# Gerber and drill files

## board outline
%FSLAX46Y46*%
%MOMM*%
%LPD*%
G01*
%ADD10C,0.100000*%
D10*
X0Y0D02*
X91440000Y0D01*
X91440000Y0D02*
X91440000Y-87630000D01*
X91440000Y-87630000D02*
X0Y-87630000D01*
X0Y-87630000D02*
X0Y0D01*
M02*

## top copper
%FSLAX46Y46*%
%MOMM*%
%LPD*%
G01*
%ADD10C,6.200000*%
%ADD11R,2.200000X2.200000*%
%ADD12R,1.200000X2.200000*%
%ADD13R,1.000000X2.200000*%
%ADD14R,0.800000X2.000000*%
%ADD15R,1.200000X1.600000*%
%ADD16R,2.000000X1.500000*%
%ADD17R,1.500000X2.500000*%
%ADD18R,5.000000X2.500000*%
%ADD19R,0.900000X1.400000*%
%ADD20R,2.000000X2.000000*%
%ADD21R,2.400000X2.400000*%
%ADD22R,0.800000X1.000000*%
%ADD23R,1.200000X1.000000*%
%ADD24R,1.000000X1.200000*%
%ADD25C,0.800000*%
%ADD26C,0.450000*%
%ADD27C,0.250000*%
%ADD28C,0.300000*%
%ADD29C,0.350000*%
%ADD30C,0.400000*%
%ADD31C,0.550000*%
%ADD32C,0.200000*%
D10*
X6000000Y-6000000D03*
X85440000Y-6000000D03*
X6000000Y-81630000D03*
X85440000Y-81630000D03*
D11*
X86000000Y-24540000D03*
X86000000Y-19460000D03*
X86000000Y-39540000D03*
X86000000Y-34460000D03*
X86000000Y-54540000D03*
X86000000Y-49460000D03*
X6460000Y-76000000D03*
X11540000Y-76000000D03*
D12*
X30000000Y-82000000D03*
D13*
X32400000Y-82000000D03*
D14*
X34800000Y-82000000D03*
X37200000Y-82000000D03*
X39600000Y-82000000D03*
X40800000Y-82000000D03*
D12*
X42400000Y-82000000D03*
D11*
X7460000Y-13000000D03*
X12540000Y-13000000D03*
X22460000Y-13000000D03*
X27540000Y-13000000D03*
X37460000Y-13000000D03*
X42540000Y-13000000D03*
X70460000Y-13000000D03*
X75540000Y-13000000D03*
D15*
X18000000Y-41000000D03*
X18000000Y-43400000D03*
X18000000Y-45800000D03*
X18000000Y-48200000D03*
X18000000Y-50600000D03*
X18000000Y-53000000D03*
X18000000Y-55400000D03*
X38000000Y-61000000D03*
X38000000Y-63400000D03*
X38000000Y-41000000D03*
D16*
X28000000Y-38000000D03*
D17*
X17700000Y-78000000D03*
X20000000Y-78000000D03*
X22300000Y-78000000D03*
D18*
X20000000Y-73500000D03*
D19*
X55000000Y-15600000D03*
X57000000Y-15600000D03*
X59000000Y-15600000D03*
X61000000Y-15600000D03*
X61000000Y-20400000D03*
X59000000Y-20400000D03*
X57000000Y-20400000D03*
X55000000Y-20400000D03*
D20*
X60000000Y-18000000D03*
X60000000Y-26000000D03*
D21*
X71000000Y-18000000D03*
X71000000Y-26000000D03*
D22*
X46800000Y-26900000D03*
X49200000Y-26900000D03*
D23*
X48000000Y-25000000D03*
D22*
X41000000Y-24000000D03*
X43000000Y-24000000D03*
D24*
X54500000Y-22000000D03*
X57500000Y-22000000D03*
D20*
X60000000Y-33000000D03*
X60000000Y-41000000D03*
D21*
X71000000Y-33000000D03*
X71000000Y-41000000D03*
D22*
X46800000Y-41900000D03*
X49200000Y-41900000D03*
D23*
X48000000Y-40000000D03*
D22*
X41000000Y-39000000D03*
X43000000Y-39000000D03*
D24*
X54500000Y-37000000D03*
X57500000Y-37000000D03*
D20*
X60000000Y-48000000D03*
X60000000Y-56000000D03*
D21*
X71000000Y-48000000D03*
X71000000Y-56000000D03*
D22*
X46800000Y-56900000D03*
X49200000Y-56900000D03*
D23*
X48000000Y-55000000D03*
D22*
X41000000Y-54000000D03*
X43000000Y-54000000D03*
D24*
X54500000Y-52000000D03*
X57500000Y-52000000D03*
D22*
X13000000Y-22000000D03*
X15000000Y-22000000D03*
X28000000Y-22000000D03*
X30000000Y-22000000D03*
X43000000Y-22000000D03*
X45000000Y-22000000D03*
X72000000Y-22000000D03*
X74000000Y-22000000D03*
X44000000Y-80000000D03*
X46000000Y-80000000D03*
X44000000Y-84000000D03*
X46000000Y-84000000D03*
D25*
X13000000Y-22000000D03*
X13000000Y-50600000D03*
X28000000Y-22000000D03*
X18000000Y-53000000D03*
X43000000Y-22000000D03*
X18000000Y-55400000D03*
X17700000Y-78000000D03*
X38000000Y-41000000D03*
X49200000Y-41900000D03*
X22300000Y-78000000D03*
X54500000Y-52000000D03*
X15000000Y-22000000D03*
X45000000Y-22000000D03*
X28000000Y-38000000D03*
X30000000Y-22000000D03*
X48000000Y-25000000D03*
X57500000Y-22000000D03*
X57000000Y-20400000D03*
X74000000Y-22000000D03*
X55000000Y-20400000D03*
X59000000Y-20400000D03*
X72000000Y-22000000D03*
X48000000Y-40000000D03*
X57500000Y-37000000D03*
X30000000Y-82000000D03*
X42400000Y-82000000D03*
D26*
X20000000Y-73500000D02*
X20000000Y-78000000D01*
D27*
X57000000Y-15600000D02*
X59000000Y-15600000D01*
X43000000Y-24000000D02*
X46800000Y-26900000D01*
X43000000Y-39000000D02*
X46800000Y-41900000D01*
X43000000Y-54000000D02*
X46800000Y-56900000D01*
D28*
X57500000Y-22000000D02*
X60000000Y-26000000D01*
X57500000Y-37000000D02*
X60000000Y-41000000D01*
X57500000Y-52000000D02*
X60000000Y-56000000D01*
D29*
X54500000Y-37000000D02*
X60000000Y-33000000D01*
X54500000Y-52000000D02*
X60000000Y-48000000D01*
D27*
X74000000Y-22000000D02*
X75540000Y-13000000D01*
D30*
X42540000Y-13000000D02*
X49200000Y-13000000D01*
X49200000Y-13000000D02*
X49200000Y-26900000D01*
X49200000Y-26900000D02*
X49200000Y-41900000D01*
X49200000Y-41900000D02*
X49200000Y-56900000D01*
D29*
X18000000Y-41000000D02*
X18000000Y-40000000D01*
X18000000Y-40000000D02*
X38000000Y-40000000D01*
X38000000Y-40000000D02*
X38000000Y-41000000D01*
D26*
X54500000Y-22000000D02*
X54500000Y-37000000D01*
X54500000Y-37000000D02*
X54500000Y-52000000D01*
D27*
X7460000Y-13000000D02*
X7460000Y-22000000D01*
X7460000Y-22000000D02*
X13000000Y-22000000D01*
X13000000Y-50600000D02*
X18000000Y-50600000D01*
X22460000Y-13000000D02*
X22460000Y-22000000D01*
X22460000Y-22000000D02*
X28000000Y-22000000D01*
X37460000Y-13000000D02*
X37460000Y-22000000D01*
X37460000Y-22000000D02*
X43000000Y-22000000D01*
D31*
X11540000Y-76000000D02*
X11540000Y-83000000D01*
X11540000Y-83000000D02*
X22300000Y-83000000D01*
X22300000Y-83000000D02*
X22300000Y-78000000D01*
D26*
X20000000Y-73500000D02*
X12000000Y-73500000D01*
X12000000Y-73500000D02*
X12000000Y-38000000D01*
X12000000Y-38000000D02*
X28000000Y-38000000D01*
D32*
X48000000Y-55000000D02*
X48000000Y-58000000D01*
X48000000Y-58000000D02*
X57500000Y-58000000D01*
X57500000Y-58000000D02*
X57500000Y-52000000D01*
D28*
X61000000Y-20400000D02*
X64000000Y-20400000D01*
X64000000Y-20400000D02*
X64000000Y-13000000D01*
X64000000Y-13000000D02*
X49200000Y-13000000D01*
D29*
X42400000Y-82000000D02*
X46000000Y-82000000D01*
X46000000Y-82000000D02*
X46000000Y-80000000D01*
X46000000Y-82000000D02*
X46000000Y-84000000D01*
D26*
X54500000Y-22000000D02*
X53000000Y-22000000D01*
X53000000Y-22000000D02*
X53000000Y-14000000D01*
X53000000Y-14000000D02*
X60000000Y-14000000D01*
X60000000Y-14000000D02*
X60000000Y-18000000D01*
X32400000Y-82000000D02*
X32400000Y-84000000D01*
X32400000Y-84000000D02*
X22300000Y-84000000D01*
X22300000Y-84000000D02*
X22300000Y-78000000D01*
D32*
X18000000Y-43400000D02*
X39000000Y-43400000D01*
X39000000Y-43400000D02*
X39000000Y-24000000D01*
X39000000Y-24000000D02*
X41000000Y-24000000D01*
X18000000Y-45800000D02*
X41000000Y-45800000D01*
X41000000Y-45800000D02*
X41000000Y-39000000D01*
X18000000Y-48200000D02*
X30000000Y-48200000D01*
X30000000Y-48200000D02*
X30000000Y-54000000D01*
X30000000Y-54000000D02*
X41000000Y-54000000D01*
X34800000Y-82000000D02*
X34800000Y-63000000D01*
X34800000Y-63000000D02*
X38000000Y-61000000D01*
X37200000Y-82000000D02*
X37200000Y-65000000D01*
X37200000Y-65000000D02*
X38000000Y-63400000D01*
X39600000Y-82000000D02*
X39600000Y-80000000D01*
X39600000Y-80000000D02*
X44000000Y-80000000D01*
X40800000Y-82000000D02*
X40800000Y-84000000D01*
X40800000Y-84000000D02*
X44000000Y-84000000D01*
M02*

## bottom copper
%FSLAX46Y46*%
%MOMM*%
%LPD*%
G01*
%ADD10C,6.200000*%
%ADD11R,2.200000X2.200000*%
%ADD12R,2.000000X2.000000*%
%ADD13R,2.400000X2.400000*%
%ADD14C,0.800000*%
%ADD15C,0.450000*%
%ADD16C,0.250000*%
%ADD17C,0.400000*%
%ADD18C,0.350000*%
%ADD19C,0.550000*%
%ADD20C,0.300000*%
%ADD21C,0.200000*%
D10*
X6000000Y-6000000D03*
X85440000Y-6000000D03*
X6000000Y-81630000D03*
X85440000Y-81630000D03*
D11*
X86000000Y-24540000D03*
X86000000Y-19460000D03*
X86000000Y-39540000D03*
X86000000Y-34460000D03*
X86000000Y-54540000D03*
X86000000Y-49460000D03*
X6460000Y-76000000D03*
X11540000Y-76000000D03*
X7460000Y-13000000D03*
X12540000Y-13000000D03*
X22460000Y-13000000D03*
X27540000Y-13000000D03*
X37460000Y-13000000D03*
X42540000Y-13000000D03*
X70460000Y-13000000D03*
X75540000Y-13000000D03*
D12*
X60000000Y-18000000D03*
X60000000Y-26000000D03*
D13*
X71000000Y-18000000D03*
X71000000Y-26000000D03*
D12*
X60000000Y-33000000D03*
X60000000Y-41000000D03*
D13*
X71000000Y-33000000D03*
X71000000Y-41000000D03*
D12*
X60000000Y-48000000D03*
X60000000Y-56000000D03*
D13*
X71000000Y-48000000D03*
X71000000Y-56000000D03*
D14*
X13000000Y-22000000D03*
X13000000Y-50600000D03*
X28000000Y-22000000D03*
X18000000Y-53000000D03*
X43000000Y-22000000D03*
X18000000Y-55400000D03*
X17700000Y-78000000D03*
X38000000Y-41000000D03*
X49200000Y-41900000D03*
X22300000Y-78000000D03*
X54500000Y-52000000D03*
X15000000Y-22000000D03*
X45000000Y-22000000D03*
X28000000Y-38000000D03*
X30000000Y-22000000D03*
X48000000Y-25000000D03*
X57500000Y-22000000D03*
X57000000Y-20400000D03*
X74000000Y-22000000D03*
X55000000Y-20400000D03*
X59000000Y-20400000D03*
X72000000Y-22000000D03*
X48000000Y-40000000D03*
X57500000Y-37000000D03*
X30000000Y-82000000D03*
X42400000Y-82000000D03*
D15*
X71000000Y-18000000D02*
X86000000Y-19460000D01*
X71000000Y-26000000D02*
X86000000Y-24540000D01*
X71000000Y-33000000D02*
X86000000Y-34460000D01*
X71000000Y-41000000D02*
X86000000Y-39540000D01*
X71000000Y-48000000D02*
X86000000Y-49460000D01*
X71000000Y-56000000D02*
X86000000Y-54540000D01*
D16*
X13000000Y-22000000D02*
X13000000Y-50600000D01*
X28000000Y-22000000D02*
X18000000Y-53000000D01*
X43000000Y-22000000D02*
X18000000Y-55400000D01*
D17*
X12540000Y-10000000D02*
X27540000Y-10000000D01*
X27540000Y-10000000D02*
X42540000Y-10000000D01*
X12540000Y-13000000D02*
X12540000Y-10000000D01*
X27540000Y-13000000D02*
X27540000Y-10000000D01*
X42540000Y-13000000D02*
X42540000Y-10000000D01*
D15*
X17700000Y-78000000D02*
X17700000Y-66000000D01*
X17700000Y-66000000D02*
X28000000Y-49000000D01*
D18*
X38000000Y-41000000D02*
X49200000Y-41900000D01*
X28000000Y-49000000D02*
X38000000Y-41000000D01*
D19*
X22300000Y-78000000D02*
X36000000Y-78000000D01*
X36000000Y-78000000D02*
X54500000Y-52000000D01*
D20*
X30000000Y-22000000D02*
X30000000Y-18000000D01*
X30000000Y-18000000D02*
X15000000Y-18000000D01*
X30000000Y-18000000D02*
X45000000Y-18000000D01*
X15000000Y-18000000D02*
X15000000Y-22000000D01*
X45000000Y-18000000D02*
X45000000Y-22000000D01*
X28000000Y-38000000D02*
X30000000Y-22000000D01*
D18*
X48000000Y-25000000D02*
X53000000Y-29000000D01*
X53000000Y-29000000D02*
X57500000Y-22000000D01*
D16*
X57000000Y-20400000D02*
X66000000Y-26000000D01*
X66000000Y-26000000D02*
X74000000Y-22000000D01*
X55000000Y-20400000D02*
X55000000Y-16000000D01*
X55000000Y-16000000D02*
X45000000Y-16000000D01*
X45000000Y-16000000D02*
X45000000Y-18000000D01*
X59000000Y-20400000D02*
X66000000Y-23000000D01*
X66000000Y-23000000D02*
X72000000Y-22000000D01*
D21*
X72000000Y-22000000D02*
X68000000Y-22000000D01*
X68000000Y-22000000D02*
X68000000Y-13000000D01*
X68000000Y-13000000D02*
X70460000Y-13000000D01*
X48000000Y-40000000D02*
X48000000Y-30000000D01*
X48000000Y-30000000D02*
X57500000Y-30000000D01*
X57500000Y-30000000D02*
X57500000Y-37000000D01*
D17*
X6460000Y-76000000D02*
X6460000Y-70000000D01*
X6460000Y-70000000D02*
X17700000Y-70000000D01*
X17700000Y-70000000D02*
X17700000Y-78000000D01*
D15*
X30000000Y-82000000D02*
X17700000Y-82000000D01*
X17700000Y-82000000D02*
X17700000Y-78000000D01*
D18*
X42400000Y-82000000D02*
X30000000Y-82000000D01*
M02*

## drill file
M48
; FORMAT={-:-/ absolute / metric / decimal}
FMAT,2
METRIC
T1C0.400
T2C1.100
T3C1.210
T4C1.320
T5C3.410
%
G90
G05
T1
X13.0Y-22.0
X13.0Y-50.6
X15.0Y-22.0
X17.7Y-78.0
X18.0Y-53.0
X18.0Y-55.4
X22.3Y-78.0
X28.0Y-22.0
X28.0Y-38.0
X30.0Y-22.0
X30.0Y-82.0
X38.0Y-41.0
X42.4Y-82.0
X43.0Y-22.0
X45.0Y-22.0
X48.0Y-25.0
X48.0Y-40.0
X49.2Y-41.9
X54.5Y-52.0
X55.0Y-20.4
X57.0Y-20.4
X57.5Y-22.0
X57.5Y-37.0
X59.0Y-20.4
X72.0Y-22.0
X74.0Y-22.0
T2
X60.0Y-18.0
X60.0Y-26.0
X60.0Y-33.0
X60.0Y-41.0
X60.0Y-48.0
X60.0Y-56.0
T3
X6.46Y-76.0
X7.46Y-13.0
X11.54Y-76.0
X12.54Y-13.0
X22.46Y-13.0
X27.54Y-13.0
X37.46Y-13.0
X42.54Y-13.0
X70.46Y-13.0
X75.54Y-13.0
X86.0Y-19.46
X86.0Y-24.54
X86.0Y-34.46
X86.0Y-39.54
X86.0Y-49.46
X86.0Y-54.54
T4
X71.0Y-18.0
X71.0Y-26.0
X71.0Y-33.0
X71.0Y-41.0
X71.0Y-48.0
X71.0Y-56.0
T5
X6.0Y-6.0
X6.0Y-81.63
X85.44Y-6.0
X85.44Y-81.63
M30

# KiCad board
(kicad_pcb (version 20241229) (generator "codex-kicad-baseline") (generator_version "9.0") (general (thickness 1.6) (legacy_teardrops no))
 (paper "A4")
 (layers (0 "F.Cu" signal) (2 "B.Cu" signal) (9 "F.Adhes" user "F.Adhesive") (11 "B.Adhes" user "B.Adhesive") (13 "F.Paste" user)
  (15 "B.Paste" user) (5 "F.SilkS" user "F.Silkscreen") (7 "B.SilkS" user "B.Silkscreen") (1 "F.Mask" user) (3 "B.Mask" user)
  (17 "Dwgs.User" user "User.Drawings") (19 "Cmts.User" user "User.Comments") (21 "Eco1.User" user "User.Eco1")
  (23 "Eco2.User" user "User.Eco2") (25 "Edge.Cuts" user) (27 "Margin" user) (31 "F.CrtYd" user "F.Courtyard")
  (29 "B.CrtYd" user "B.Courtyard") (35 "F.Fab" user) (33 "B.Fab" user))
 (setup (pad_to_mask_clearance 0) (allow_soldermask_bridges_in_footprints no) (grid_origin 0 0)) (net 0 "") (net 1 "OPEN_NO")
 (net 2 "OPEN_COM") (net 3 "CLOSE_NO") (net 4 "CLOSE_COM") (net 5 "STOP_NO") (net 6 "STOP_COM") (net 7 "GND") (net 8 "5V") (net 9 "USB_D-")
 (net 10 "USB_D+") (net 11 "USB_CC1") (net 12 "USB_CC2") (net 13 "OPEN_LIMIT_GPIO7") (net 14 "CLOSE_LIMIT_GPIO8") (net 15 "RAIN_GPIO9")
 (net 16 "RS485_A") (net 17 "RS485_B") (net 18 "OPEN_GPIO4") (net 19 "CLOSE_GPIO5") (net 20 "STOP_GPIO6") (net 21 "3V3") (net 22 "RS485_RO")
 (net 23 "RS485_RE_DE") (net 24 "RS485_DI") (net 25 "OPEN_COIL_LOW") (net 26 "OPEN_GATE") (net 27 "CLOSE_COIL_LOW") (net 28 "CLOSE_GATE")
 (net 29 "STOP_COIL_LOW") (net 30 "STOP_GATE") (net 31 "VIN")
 (gr_line (start 0.00 0.00) (end 91.44 0.00) (stroke (width 0.1) (type solid)) (layer "Edge.Cuts"))
 (gr_line (start 91.44 0.00) (end 91.44 87.63) (stroke (width 0.1) (type solid)) (layer "Edge.Cuts"))
 (gr_line (start 91.44 87.63) (end 0.00 87.63) (stroke (width 0.1) (type solid)) (layer "Edge.Cuts"))
 (gr_line (start 0.00 87.63) (end 0.00 0.00) (stroke (width 0.1) (type solid)) (layer "Edge.Cuts"))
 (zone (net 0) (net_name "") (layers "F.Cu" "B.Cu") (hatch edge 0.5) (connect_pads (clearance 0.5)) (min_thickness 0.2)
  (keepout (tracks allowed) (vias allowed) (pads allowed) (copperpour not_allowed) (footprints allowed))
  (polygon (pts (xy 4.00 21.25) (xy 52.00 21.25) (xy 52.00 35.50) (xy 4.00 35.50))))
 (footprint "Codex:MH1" (layer "F.Cu") (at 6.00 6.00 0)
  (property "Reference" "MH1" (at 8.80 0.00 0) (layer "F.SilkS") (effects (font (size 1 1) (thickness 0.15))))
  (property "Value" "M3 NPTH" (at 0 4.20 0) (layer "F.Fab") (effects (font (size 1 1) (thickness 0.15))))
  (pad "1" np_thru_hole circle (at 0.00 0.00) (size 6.20 6.20) (drill 3.41) (layers "*.Cu" "*.Mask")))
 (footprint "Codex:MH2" (layer "F.Cu") (at 85.44 6.00 0)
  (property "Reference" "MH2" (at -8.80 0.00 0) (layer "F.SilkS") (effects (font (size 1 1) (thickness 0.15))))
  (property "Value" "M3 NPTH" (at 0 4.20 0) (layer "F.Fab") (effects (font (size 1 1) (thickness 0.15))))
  (pad "1" np_thru_hole circle (at 0.00 0.00) (size 6.20 6.20) (drill 3.41) (layers "*.Cu" "*.Mask")))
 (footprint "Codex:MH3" (layer "F.Cu") (at 6.00 81.63 0)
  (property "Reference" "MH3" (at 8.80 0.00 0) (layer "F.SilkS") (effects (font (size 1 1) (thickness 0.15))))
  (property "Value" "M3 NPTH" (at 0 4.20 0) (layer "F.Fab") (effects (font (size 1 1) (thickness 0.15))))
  (pad "1" np_thru_hole circle (at 0.00 0.00) (size 6.20 6.20) (drill 3.41) (layers "*.Cu" "*.Mask")))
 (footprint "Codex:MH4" (layer "F.Cu") (at 85.44 81.63 0)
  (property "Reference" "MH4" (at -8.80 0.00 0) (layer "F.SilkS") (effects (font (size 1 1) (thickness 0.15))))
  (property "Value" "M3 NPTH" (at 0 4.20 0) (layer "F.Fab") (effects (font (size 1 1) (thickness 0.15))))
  (pad "1" np_thru_hole circle (at 0.00 0.00) (size 6.20 6.20) (drill 3.41) (layers "*.Cu" "*.Mask")))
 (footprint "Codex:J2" (layer "F.Cu") (at 86.00 22.00 90)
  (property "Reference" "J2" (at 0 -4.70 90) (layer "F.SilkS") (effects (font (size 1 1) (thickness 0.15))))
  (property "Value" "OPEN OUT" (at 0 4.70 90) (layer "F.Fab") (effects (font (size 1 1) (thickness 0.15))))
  (pad "1" thru_hole rect (at -2.54 0.00) (size 2.20 2.20) (drill 1.21) (layers "*.Cu" "*.Mask") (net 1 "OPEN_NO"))
  (pad "2" thru_hole rect (at 2.54 0.00) (size 2.20 2.20) (drill 1.21) (layers "*.Cu" "*.Mask") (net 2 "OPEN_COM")))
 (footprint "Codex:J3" (layer "F.Cu") (at 86.00 37.00 90)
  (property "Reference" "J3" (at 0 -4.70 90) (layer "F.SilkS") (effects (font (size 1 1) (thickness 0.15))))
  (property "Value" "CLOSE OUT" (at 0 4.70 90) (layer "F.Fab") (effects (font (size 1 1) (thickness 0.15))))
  (pad "1" thru_hole rect (at -2.54 0.00) (size 2.20 2.20) (drill 1.21) (layers "*.Cu" "*.Mask") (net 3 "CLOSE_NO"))
  (pad "2" thru_hole rect (at 2.54 0.00) (size 2.20 2.20) (drill 1.21) (layers "*.Cu" "*.Mask") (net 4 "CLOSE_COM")))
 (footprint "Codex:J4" (layer "F.Cu") (at 86.00 52.00 90)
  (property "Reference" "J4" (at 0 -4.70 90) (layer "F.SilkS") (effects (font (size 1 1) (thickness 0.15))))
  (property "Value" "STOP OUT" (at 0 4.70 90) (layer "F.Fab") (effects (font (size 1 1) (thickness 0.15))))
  (pad "1" thru_hole rect (at -2.54 0.00) (size 2.20 2.20) (drill 1.21) (layers "*.Cu" "*.Mask") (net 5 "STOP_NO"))
  (pad "2" thru_hole rect (at 2.54 0.00) (size 2.20 2.20) (drill 1.21) (layers "*.Cu" "*.Mask") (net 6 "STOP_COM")))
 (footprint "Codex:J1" (layer "F.Cu") (at 9.00 76.00 0)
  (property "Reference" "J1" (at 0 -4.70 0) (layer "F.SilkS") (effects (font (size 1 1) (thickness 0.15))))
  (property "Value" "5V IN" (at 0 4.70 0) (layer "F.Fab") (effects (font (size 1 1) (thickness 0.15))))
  (pad "1" thru_hole rect (at -2.54 0.00) (size 2.20 2.20) (drill 1.21) (layers "*.Cu" "*.Mask") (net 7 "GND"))
  (pad "2" thru_hole rect (at 2.54 0.00) (size 2.20 2.20) (drill 1.21) (layers "*.Cu" "*.Mask") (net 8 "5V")))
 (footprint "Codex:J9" (layer "F.Cu") (at 36.00 82.00 0)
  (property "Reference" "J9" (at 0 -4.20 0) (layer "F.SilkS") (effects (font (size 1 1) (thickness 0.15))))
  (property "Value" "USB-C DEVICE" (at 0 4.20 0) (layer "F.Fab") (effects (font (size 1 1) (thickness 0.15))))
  (pad "GND1" smd rect (at -6.00 0.00) (size 1.20 2.20) (layers "F.Cu" "F.Paste" "F.Mask") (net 7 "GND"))
  (pad "VBUS" smd rect (at -3.60 0.00) (size 1.00 2.20) (layers "F.Cu" "F.Paste" "F.Mask") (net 8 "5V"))
  (pad "D-" smd rect (at -1.20 0.00) (size 0.80 2.00) (layers "F.Cu" "F.Paste" "F.Mask") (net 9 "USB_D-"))
  (pad "D+" smd rect (at 1.20 0.00) (size 0.80 2.00) (layers "F.Cu" "F.Paste" "F.Mask") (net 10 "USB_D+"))
  (pad "CC1" smd rect (at 3.60 0.00) (size 0.80 2.00) (layers "F.Cu" "F.Paste" "F.Mask") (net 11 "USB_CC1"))
  (pad "CC2" smd rect (at 4.80 0.00) (size 0.80 2.00) (layers "F.Cu" "F.Paste" "F.Mask") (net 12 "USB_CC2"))
  (pad "GND2" smd rect (at 6.40 0.00) (size 1.20 2.20) (layers "F.Cu" "F.Paste" "F.Mask") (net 7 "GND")))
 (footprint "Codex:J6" (layer "F.Cu") (at 10.00 13.00 0)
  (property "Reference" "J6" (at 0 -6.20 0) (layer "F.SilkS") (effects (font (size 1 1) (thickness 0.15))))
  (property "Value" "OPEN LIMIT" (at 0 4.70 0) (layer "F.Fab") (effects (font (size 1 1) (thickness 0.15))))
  (pad "1" thru_hole rect (at -2.54 0.00) (size 2.20 2.20) (drill 1.21) (layers "*.Cu" "*.Mask") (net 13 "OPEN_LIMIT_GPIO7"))
  (pad "2" thru_hole rect (at 2.54 0.00) (size 2.20 2.20) (drill 1.21) (layers "*.Cu" "*.Mask") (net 7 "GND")))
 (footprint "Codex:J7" (layer "F.Cu") (at 25.00 13.00 0)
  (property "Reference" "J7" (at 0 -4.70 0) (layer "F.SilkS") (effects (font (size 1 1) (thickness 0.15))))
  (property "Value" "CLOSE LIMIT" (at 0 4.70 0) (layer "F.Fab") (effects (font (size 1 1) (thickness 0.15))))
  (pad "1" thru_hole rect (at -2.54 0.00) (size 2.20 2.20) (drill 1.21) (layers "*.Cu" "*.Mask") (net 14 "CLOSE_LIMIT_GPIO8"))
  (pad "2" thru_hole rect (at 2.54 0.00) (size 2.20 2.20) (drill 1.21) (layers "*.Cu" "*.Mask") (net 7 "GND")))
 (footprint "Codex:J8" (layer "F.Cu") (at 40.00 13.00 0)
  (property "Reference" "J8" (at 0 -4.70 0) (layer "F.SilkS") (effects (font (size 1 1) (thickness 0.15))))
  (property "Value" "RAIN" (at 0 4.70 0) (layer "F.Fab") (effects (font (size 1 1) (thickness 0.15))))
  (pad "1" thru_hole rect (at -2.54 0.00) (size 2.20 2.20) (drill 1.21) (layers "*.Cu" "*.Mask") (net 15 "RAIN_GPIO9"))
  (pad "2" thru_hole rect (at 2.54 0.00) (size 2.20 2.20) (drill 1.21) (layers "*.Cu" "*.Mask") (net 7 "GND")))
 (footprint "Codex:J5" (layer "F.Cu") (at 73.00 13.00 0)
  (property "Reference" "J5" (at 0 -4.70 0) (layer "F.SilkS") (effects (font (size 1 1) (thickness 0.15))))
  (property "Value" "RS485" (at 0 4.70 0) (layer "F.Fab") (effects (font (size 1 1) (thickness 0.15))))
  (pad "1" thru_hole rect (at -2.54 0.00) (size 2.20 2.20) (drill 1.21) (layers "*.Cu" "*.Mask") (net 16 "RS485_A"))
  (pad "2" thru_hole rect (at 2.54 0.00) (size 2.20 2.20) (drill 1.21) (layers "*.Cu" "*.Mask") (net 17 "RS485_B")))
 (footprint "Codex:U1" (layer "F.Cu") (at 28.00 49.00 0)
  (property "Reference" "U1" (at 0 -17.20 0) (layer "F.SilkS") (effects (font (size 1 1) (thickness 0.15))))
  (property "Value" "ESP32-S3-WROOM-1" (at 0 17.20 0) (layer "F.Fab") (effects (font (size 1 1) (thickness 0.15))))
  (pad "1" smd rect (at -10.00 -8.00) (size 1.20 1.60) (layers "F.Cu" "F.Paste" "F.Mask") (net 7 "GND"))
  (pad "4" smd rect (at -10.00 -5.60) (size 1.20 1.60) (layers "F.Cu" "F.Paste" "F.Mask") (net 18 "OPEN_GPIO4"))
  (pad "5" smd rect (at -10.00 -3.20) (size 1.20 1.60) (layers "F.Cu" "F.Paste" "F.Mask") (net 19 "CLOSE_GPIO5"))
  (pad "6" smd rect (at -10.00 -0.80) (size 1.20 1.60) (layers "F.Cu" "F.Paste" "F.Mask") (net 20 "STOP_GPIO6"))
  (pad "7" smd rect (at -10.00 1.60) (size 1.20 1.60) (layers "F.Cu" "F.Paste" "F.Mask") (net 13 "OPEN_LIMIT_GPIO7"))
  (pad "12" smd rect (at -10.00 4.00) (size 1.20 1.60) (layers "F.Cu" "F.Paste" "F.Mask") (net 14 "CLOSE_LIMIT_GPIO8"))
  (pad "17" smd rect (at -10.00 6.40) (size 1.20 1.60) (layers "F.Cu" "F.Paste" "F.Mask") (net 15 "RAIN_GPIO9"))
  (pad "19" smd rect (at 10.00 12.00) (size 1.20 1.60) (layers "F.Cu" "F.Paste" "F.Mask") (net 9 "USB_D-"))
  (pad "20" smd rect (at 10.00 14.40) (size 1.20 1.60) (layers "F.Cu" "F.Paste" "F.Mask") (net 10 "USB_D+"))
  (pad "40" smd rect (at 10.00 -8.00) (size 1.20 1.60) (layers "F.Cu" "F.Paste" "F.Mask") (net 7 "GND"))
  (pad "3V3" smd rect (at 0.00 -11.00) (size 2.00 1.50) (layers "F.Cu" "F.Paste" "F.Mask") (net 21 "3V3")))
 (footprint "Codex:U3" (layer "F.Cu") (at 20.00 76.00 0)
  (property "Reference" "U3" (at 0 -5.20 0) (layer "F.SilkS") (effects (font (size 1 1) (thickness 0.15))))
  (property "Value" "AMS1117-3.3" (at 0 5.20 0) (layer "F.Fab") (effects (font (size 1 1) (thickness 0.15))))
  (pad "1" smd rect (at -2.30 2.00) (size 1.50 2.50) (layers "F.Cu" "F.Paste" "F.Mask") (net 7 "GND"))
  (pad "2" smd rect (at 0.00 2.00) (size 1.50 2.50) (layers "F.Cu" "F.Paste" "F.Mask") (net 21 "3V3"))
  (pad "3" smd rect (at 2.30 2.00) (size 1.50 2.50) (layers "F.Cu" "F.Paste" "F.Mask") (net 8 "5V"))
  (pad "4" smd rect (at 0.00 -2.50) (size 5.00 2.50) (layers "F.Cu" "F.Paste" "F.Mask") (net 21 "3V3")))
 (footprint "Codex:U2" (layer "F.Cu") (at 58.00 18.00 0)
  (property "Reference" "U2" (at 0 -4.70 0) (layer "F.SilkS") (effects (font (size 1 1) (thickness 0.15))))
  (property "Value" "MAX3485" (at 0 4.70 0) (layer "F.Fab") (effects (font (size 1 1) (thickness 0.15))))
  (pad "1" smd rect (at -3.00 -2.40) (size 0.90 1.40) (layers "F.Cu" "F.Paste" "F.Mask") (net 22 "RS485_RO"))
  (pad "2" smd rect (at -1.00 -2.40) (size 0.90 1.40) (layers "F.Cu" "F.Paste" "F.Mask") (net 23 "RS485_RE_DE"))
  (pad "3" smd rect (at 1.00 -2.40) (size 0.90 1.40) (layers "F.Cu" "F.Paste" "F.Mask") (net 23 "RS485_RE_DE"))
  (pad "4" smd rect (at 3.00 -2.40) (size 0.90 1.40) (layers "F.Cu" "F.Paste" "F.Mask") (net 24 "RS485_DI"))
  (pad "5" smd rect (at 3.00 2.40) (size 0.90 1.40) (layers "F.Cu" "F.Paste" "F.Mask") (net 7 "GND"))
  (pad "6" smd rect (at 1.00 2.40) (size 0.90 1.40) (layers "F.Cu" "F.Paste" "F.Mask") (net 16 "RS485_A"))
  (pad "7" smd rect (at -1.00 2.40) (size 0.90 1.40) (layers "F.Cu" "F.Paste" "F.Mask") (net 17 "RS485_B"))
  (pad "8" smd rect (at -3.00 2.40) (size 0.90 1.40) (layers "F.Cu" "F.Paste" "F.Mask") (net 21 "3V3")))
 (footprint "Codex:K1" (layer "F.Cu") (at 66.00 22.00 0)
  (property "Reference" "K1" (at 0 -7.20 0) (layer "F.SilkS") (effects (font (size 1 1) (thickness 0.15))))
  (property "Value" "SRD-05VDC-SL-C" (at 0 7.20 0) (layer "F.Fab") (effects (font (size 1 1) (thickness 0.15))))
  (pad "COIL+" thru_hole rect (at -6.00 -4.00) (size 2.00 2.00) (drill 1.10) (layers "*.Cu" "*.Mask") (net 8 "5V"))
  (pad "COIL-" thru_hole rect (at -6.00 4.00) (size 2.00 2.00) (drill 1.10) (layers "*.Cu" "*.Mask") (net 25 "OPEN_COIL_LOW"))
  (pad "COM" thru_hole rect (at 5.00 -4.00) (size 2.40 2.40) (drill 1.32) (layers "*.Cu" "*.Mask") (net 2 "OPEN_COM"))
  (pad "NO" thru_hole rect (at 5.00 4.00) (size 2.40 2.40) (drill 1.32) (layers "*.Cu" "*.Mask") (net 1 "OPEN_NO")))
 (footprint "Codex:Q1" (layer "F.Cu") (at 48.00 26.00 0)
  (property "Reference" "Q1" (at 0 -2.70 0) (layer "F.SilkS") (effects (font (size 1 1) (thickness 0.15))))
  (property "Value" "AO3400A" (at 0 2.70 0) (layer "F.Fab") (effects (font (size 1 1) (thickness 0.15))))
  (pad "1" smd rect (at -1.20 0.90) (size 0.80 1.00) (layers "F.Cu" "F.Paste" "F.Mask") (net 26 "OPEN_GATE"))
  (pad "2" smd rect (at 1.20 0.90) (size 0.80 1.00) (layers "F.Cu" "F.Paste" "F.Mask") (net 7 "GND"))
  (pad "3" smd rect (at 0.00 -1.00) (size 1.20 1.00) (layers "F.Cu" "F.Paste" "F.Mask") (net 25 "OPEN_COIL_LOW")))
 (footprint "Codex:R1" (layer "F.Cu") (at 42.00 24.00 0)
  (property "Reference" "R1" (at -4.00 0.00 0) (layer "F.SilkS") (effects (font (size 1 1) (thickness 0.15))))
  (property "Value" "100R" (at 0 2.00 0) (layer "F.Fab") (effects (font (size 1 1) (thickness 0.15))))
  (pad "1" smd rect (at -1.00 0.00) (size 0.80 1.00) (layers "F.Cu" "F.Paste" "F.Mask") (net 18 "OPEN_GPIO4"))
  (pad "2" smd rect (at 1.00 0.00) (size 0.80 1.00) (layers "F.Cu" "F.Paste" "F.Mask") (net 26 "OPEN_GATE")))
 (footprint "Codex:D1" (layer "F.Cu") (at 56.00 22.00 0)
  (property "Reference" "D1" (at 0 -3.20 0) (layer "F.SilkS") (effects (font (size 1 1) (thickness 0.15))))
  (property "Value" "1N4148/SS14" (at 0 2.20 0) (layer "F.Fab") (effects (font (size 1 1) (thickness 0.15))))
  (pad "1" smd rect (at -1.50 0.00) (size 1.00 1.20) (layers "F.Cu" "F.Paste" "F.Mask") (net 8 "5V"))
  (pad "2" smd rect (at 1.50 0.00) (size 1.00 1.20) (layers "F.Cu" "F.Paste" "F.Mask") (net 25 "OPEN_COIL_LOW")))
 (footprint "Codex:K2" (layer "F.Cu") (at 66.00 37.00 0)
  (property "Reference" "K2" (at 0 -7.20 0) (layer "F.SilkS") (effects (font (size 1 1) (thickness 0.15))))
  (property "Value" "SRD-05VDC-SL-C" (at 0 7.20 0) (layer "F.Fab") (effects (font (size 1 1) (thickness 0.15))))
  (pad "COIL+" thru_hole rect (at -6.00 -4.00) (size 2.00 2.00) (drill 1.10) (layers "*.Cu" "*.Mask") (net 8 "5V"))
  (pad "COIL-" thru_hole rect (at -6.00 4.00) (size 2.00 2.00) (drill 1.10) (layers "*.Cu" "*.Mask") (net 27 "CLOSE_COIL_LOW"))
  (pad "COM" thru_hole rect (at 5.00 -4.00) (size 2.40 2.40) (drill 1.32) (layers "*.Cu" "*.Mask") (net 4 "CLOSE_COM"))
  (pad "NO" thru_hole rect (at 5.00 4.00) (size 2.40 2.40) (drill 1.32) (layers "*.Cu" "*.Mask") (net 3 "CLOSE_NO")))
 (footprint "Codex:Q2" (layer "F.Cu") (at 48.00 41.00 0)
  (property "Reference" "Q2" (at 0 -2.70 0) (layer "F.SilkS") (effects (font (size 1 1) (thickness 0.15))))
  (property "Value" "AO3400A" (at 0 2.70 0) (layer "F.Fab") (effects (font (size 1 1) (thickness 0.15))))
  (pad "1" smd rect (at -1.20 0.90) (size 0.80 1.00) (layers "F.Cu" "F.Paste" "F.Mask") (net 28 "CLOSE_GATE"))
  (pad "2" smd rect (at 1.20 0.90) (size 0.80 1.00) (layers "F.Cu" "F.Paste" "F.Mask") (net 7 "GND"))
  (pad "3" smd rect (at 0.00 -1.00) (size 1.20 1.00) (layers "F.Cu" "F.Paste" "F.Mask") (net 27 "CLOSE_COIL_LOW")))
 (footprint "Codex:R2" (layer "F.Cu") (at 42.00 39.00 0)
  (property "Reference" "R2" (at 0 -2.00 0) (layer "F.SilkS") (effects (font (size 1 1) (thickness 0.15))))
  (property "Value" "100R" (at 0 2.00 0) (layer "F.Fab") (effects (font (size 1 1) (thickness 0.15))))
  (pad "1" smd rect (at -1.00 0.00) (size 0.80 1.00) (layers "F.Cu" "F.Paste" "F.Mask") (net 19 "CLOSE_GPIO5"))
  (pad "2" smd rect (at 1.00 0.00) (size 0.80 1.00) (layers "F.Cu" "F.Paste" "F.Mask") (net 28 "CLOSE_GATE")))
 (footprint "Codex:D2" (layer "F.Cu") (at 56.00 37.00 0)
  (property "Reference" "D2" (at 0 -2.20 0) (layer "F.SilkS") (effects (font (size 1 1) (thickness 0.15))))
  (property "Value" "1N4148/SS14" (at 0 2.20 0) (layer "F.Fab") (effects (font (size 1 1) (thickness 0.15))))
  (pad "1" smd rect (at -1.50 0.00) (size 1.00 1.20) (layers "F.Cu" "F.Paste" "F.Mask") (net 8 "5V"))
  (pad "2" smd rect (at 1.50 0.00) (size 1.00 1.20) (layers "F.Cu" "F.Paste" "F.Mask") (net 27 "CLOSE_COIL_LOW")))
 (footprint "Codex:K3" (layer "F.Cu") (at 66.00 52.00 0)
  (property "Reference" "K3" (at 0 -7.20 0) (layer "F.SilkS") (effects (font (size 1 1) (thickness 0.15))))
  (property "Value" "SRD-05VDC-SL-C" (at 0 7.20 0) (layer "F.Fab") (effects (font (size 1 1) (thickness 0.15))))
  (pad "COIL+" thru_hole rect (at -6.00 -4.00) (size 2.00 2.00) (drill 1.10) (layers "*.Cu" "*.Mask") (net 8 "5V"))
  (pad "COIL-" thru_hole rect (at -6.00 4.00) (size 2.00 2.00) (drill 1.10) (layers "*.Cu" "*.Mask") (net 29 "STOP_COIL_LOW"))
  (pad "COM" thru_hole rect (at 5.00 -4.00) (size 2.40 2.40) (drill 1.32) (layers "*.Cu" "*.Mask") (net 6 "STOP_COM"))
  (pad "NO" thru_hole rect (at 5.00 4.00) (size 2.40 2.40) (drill 1.32) (layers "*.Cu" "*.Mask") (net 5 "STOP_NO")))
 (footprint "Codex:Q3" (layer "F.Cu") (at 48.00 56.00 0)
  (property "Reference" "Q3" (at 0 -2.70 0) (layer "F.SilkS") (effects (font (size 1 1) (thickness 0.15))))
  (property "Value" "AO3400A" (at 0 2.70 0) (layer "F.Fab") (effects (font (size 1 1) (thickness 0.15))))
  (pad "1" smd rect (at -1.20 0.90) (size 0.80 1.00) (layers "F.Cu" "F.Paste" "F.Mask") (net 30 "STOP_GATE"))
  (pad "2" smd rect (at 1.20 0.90) (size 0.80 1.00) (layers "F.Cu" "F.Paste" "F.Mask") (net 7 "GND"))
  (pad "3" smd rect (at 0.00 -1.00) (size 1.20 1.00) (layers "F.Cu" "F.Paste" "F.Mask") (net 29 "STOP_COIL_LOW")))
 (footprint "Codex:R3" (layer "F.Cu") (at 42.00 54.00 0)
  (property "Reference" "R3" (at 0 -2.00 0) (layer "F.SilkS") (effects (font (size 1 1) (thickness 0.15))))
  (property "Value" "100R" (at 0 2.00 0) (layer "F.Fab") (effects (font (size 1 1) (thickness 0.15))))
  (pad "1" smd rect (at -1.00 0.00) (size 0.80 1.00) (layers "F.Cu" "F.Paste" "F.Mask") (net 20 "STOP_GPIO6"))
  (pad "2" smd rect (at 1.00 0.00) (size 0.80 1.00) (layers "F.Cu" "F.Paste" "F.Mask") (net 30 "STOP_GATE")))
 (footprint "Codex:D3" (layer "F.Cu") (at 56.00 52.00 0)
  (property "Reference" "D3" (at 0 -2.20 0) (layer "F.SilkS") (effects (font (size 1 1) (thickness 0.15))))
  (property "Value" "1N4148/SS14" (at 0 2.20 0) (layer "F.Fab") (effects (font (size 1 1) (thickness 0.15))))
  (pad "1" smd rect (at -1.50 0.00) (size 1.00 1.20) (layers "F.Cu" "F.Paste" "F.Mask") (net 8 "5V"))
  (pad "2" smd rect (at 1.50 0.00) (size 1.00 1.20) (layers "F.Cu" "F.Paste" "F.Mask") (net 29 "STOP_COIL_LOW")))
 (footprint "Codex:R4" (layer "F.Cu") (at 14.00 22.00 0)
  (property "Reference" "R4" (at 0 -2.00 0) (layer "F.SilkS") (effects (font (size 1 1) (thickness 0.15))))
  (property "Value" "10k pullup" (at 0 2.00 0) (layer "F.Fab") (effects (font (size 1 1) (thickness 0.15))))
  (pad "1" smd rect (at -1.00 0.00) (size 0.80 1.00) (layers "F.Cu" "F.Paste" "F.Mask") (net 13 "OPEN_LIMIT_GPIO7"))
  (pad "2" smd rect (at 1.00 0.00) (size 0.80 1.00) (layers "F.Cu" "F.Paste" "F.Mask") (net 21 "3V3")))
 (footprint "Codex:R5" (layer "F.Cu") (at 29.00 22.00 0)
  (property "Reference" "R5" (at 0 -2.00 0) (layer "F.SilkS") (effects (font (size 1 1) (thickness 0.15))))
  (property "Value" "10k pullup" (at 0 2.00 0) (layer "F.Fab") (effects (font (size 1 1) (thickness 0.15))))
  (pad "1" smd rect (at -1.00 0.00) (size 0.80 1.00) (layers "F.Cu" "F.Paste" "F.Mask") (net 14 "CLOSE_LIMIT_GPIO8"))
  (pad "2" smd rect (at 1.00 0.00) (size 0.80 1.00) (layers "F.Cu" "F.Paste" "F.Mask") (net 21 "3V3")))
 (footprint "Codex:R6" (layer "F.Cu") (at 44.00 22.00 0)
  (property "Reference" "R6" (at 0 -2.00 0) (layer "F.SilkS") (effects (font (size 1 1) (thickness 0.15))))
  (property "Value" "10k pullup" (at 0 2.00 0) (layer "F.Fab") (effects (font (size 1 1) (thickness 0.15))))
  (pad "1" smd rect (at -1.00 0.00) (size 0.80 1.00) (layers "F.Cu" "F.Paste" "F.Mask") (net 15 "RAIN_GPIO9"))
  (pad "2" smd rect (at 1.00 0.00) (size 0.80 1.00) (layers "F.Cu" "F.Paste" "F.Mask") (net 21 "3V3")))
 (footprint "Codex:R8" (layer "F.Cu") (at 73.00 22.00 0)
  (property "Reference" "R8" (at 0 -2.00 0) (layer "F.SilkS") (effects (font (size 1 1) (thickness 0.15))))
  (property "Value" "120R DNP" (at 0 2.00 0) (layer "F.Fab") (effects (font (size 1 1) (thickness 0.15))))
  (pad "1" smd rect (at -1.00 0.00) (size 0.80 1.00) (layers "F.Cu" "F.Paste" "F.Mask") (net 16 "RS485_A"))
  (pad "2" smd rect (at 1.00 0.00) (size 0.80 1.00) (layers "F.Cu" "F.Paste" "F.Mask") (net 17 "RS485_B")))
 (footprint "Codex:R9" (layer "F.Cu") (at 45.00 80.00 0)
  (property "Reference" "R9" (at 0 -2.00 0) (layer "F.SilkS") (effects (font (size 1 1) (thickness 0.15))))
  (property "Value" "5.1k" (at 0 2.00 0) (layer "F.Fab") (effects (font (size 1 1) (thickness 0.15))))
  (pad "1" smd rect (at -1.00 0.00) (size 0.80 1.00) (layers "F.Cu" "F.Paste" "F.Mask") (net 11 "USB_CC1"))
  (pad "2" smd rect (at 1.00 0.00) (size 0.80 1.00) (layers "F.Cu" "F.Paste" "F.Mask") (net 7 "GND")))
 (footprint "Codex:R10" (layer "F.Cu") (at 45.00 84.00 0)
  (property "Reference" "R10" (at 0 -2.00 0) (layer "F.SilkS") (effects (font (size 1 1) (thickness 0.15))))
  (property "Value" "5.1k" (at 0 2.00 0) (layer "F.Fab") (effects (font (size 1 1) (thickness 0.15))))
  (pad "1" smd rect (at -1.00 0.00) (size 0.80 1.00) (layers "F.Cu" "F.Paste" "F.Mask") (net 12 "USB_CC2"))
  (pad "2" smd rect (at 1.00 0.00) (size 0.80 1.00) (layers "F.Cu" "F.Paste" "F.Mask") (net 7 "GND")))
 (segment (start 71.00 18.00) (end 86.00 19.46) (width 0.45) (layer "B.Cu") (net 2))
 (segment (start 71.00 26.00) (end 86.00 24.54) (width 0.45) (layer "B.Cu") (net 1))
 (segment (start 71.00 33.00) (end 86.00 34.46) (width 0.45) (layer "B.Cu") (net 4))
 (segment (start 71.00 41.00) (end 86.00 39.54) (width 0.45) (layer "B.Cu") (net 3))
 (segment (start 71.00 48.00) (end 86.00 49.46) (width 0.45) (layer "B.Cu") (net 6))
 (segment (start 71.00 56.00) (end 86.00 54.54) (width 0.45) (layer "B.Cu") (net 5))
 (segment (start 20.00 73.50) (end 20.00 78.00) (width 0.45) (layer "F.Cu") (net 21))
 (segment (start 57.00 15.60) (end 59.00 15.60) (width 0.25) (layer "F.Cu") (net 23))
 (segment (start 43.00 24.00) (end 46.80 26.90) (width 0.25) (layer "F.Cu") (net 26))
 (segment (start 43.00 39.00) (end 46.80 41.90) (width 0.25) (layer "F.Cu") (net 28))
 (segment (start 43.00 54.00) (end 46.80 56.90) (width 0.25) (layer "F.Cu") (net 30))
 (segment (start 57.50 22.00) (end 60.00 26.00) (width 0.30) (layer "F.Cu") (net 25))
 (segment (start 57.50 37.00) (end 60.00 41.00) (width 0.30) (layer "F.Cu") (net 27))
 (segment (start 57.50 52.00) (end 60.00 56.00) (width 0.30) (layer "F.Cu") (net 29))
 (segment (start 54.50 37.00) (end 60.00 33.00) (width 0.35) (layer "F.Cu") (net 8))
 (segment (start 54.50 52.00) (end 60.00 48.00) (width 0.35) (layer "F.Cu") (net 8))
 (segment (start 74.00 22.00) (end 75.54 13.00) (width 0.25) (layer "F.Cu") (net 17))
 (segment (start 42.54 13.00) (end 49.20 13.00) (width 0.40) (layer "F.Cu") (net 7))
 (segment (start 49.20 13.00) (end 49.20 26.90) (width 0.40) (layer "F.Cu") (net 7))
 (segment (start 49.20 26.90) (end 49.20 41.90) (width 0.40) (layer "F.Cu") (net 7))
 (segment (start 49.20 41.90) (end 49.20 56.90) (width 0.40) (layer "F.Cu") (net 7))
 (segment (start 18.00 41.00) (end 18.00 40.00) (width 0.35) (layer "F.Cu") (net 7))
 (segment (start 18.00 40.00) (end 38.00 40.00) (width 0.35) (layer "F.Cu") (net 7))
 (segment (start 38.00 40.00) (end 38.00 41.00) (width 0.35) (layer "F.Cu") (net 7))
 (segment (start 54.50 22.00) (end 54.50 37.00) (width 0.45) (layer "F.Cu") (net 8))
 (segment (start 54.50 37.00) (end 54.50 52.00) (width 0.45) (layer "F.Cu") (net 8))
 (segment (start 7.46 13.00) (end 7.46 22.00) (width 0.25) (layer "F.Cu") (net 13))
 (segment (start 7.46 22.00) (end 13.00 22.00) (width 0.25) (layer "F.Cu") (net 13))
 (segment (start 13.00 22.00) (end 13.00 50.60) (width 0.25) (layer "B.Cu") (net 13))
 (via (at 13.00 22.00) (size 0.80) (drill 0.40) (layers "F.Cu" "B.Cu") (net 13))
 (via (at 13.00 50.60) (size 0.80) (drill 0.40) (layers "F.Cu" "B.Cu") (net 13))
 (segment (start 13.00 50.60) (end 18.00 50.60) (width 0.25) (layer "F.Cu") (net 13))
 (segment (start 22.46 13.00) (end 22.46 22.00) (width 0.25) (layer "F.Cu") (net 14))
 (segment (start 22.46 22.00) (end 28.00 22.00) (width 0.25) (layer "F.Cu") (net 14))
 (segment (start 28.00 22.00) (end 18.00 53.00) (width 0.25) (layer "B.Cu") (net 14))
 (via (at 28.00 22.00) (size 0.80) (drill 0.40) (layers "F.Cu" "B.Cu") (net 14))
 (via (at 18.00 53.00) (size 0.80) (drill 0.40) (layers "F.Cu" "B.Cu") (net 14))
 (segment (start 37.46 13.00) (end 37.46 22.00) (width 0.25) (layer "F.Cu") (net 15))
 (segment (start 37.46 22.00) (end 43.00 22.00) (width 0.25) (layer "F.Cu") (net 15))
 (segment (start 43.00 22.00) (end 18.00 55.40) (width 0.25) (layer "B.Cu") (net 15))
 (via (at 43.00 22.00) (size 0.80) (drill 0.40) (layers "F.Cu" "B.Cu") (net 15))
 (via (at 18.00 55.40) (size 0.80) (drill 0.40) (layers "F.Cu" "B.Cu") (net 15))
 (segment (start 12.54 10.00) (end 27.54 10.00) (width 0.40) (layer "B.Cu") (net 7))
 (segment (start 27.54 10.00) (end 42.54 10.00) (width 0.40) (layer "B.Cu") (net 7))
 (segment (start 12.54 13.00) (end 12.54 10.00) (width 0.40) (layer "B.Cu") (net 7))
 (segment (start 27.54 13.00) (end 27.54 10.00) (width 0.40) (layer "B.Cu") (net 7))
 (segment (start 42.54 13.00) (end 42.54 10.00) (width 0.40) (layer "B.Cu") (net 7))
 (via (at 17.70 78.00) (size 0.80) (drill 0.40) (layers "F.Cu" "B.Cu") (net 7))
 (segment (start 17.70 78.00) (end 17.70 66.00) (width 0.45) (layer "B.Cu") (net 7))
 (segment (start 17.70 66.00) (end 28.00 49.00) (width 0.45) (layer "B.Cu") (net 7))
 (via (at 38.00 41.00) (size 0.80) (drill 0.40) (layers "F.Cu" "B.Cu") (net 7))
 (segment (start 38.00 41.00) (end 49.20 41.90) (width 0.35) (layer "B.Cu") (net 7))
 (via (at 49.20 41.90) (size 0.80) (drill 0.40) (layers "F.Cu" "B.Cu") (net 7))
 (segment (start 28.00 49.00) (end 38.00 41.00) (width 0.35) (layer "B.Cu") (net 7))
 (segment (start 11.54 76.00) (end 11.54 83.00) (width 0.55) (layer "F.Cu") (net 8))
 (segment (start 11.54 83.00) (end 22.30 83.00) (width 0.55) (layer "F.Cu") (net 8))
 (segment (start 22.30 83.00) (end 22.30 78.00) (width 0.55) (layer "F.Cu") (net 8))
 (via (at 22.30 78.00) (size 0.80) (drill 0.40) (layers "F.Cu" "B.Cu") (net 8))
 (segment (start 22.30 78.00) (end 36.00 78.00) (width 0.55) (layer "B.Cu") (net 8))
 (segment (start 36.00 78.00) (end 54.50 52.00) (width 0.55) (layer "B.Cu") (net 8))
 (via (at 54.50 52.00) (size 0.80) (drill 0.40) (layers "F.Cu" "B.Cu") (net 8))
 (segment (start 30.00 22.00) (end 30.00 18.00) (width 0.30) (layer "B.Cu") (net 21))
 (segment (start 30.00 18.00) (end 15.00 18.00) (width 0.30) (layer "B.Cu") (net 21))
 (segment (start 30.00 18.00) (end 45.00 18.00) (width 0.30) (layer "B.Cu") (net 21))
 (via (at 15.00 22.00) (size 0.80) (drill 0.40) (layers "F.Cu" "B.Cu") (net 21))
 (segment (start 15.00 18.00) (end 15.00 22.00) (width 0.30) (layer "B.Cu") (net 21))
 (via (at 45.00 22.00) (size 0.80) (drill 0.40) (layers "F.Cu" "B.Cu") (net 21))
 (segment (start 45.00 18.00) (end 45.00 22.00) (width 0.30) (layer "B.Cu") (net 21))
 (via (at 28.00 38.00) (size 0.80) (drill 0.40) (layers "F.Cu" "B.Cu") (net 21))
 (segment (start 28.00 38.00) (end 30.00 22.00) (width 0.30) (layer "B.Cu") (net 21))
 (via (at 30.00 22.00) (size 0.80) (drill 0.40) (layers "F.Cu" "B.Cu") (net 21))
 (via (at 48.00 25.00) (size 0.80) (drill 0.40) (layers "F.Cu" "B.Cu") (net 25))
 (segment (start 48.00 25.00) (end 53.00 29.00) (width 0.35) (layer "B.Cu") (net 25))
 (segment (start 53.00 29.00) (end 57.50 22.00) (width 0.35) (layer "B.Cu") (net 25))
 (via (at 57.50 22.00) (size 0.80) (drill 0.40) (layers "F.Cu" "B.Cu") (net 25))
 (via (at 57.00 20.40) (size 0.80) (drill 0.40) (layers "F.Cu" "B.Cu") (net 17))
 (segment (start 57.00 20.40) (end 66.00 26.00) (width 0.25) (layer "B.Cu") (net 17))
 (segment (start 66.00 26.00) (end 74.00 22.00) (width 0.25) (layer "B.Cu") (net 17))
 (via (at 74.00 22.00) (size 0.80) (drill 0.40) (layers "F.Cu" "B.Cu") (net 17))
 (segment (start 20.00 73.50) (end 12.00 73.50) (width 0.45) (layer "F.Cu") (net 21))
 (segment (start 12.00 73.50) (end 12.00 38.00) (width 0.45) (layer "F.Cu") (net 21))
 (segment (start 12.00 38.00) (end 28.00 38.00) (width 0.45) (layer "F.Cu") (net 21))
 (via (at 55.00 20.40) (size 0.80) (drill 0.40) (layers "F.Cu" "B.Cu") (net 21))
 (segment (start 55.00 20.40) (end 55.00 16.00) (width 0.25) (layer "B.Cu") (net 21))
 (segment (start 55.00 16.00) (end 45.00 16.00) (width 0.25) (layer "B.Cu") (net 21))
 (segment (start 45.00 16.00) (end 45.00 18.00) (width 0.25) (layer "B.Cu") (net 21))
 (via (at 59.00 20.40) (size 0.80) (drill 0.40) (layers "F.Cu" "B.Cu") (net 16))
 (segment (start 59.00 20.40) (end 66.00 23.00) (width 0.25) (layer "B.Cu") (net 16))
 (segment (start 66.00 23.00) (end 72.00 22.00) (width 0.25) (layer "B.Cu") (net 16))
 (via (at 72.00 22.00) (size 0.80) (drill 0.40) (layers "F.Cu" "B.Cu") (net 16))
 (segment (start 72.00 22.00) (end 68.00 22.00) (width 0.20) (layer "B.Cu") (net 16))
 (segment (start 68.00 22.00) (end 68.00 13.00) (width 0.20) (layer "B.Cu") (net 16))
 (segment (start 68.00 13.00) (end 70.46 13.00) (width 0.20) (layer "B.Cu") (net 16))
 (via (at 48.00 40.00) (size 0.80) (drill 0.40) (layers "F.Cu" "B.Cu") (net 27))
 (via (at 57.50 37.00) (size 0.80) (drill 0.40) (layers "F.Cu" "B.Cu") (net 27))
 (segment (start 48.00 40.00) (end 48.00 30.00) (width 0.20) (layer "B.Cu") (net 27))
 (segment (start 48.00 30.00) (end 57.50 30.00) (width 0.20) (layer "B.Cu") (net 27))
 (segment (start 57.50 30.00) (end 57.50 37.00) (width 0.20) (layer "B.Cu") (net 27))
 (segment (start 48.00 55.00) (end 48.00 58.00) (width 0.20) (layer "F.Cu") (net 29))
 (segment (start 48.00 58.00) (end 57.50 58.00) (width 0.20) (layer "F.Cu") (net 29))
 (segment (start 57.50 58.00) (end 57.50 52.00) (width 0.20) (layer "F.Cu") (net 29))
 (segment (start 6.46 76.00) (end 6.46 70.00) (width 0.40) (layer "B.Cu") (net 7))
 (segment (start 6.46 70.00) (end 17.70 70.00) (width 0.40) (layer "B.Cu") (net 7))
 (segment (start 17.70 70.00) (end 17.70 78.00) (width 0.40) (layer "B.Cu") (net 7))
 (segment (start 61.00 20.40) (end 64.00 20.40) (width 0.30) (layer "F.Cu") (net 7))
 (segment (start 64.00 20.40) (end 64.00 13.00) (width 0.30) (layer "F.Cu") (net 7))
 (segment (start 64.00 13.00) (end 49.20 13.00) (width 0.30) (layer "F.Cu") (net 7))
 (segment (start 30.00 82.00) (end 17.70 82.00) (width 0.45) (layer "B.Cu") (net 7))
 (segment (start 17.70 82.00) (end 17.70 78.00) (width 0.45) (layer "B.Cu") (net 7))
 (via (at 30.00 82.00) (size 0.80) (drill 0.40) (layers "F.Cu" "B.Cu") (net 7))
 (via (at 42.40 82.00) (size 0.80) (drill 0.40) (layers "F.Cu" "B.Cu") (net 7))
 (segment (start 42.40 82.00) (end 30.00 82.00) (width 0.35) (layer "B.Cu") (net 7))
 (segment (start 42.40 82.00) (end 46.00 82.00) (width 0.35) (layer "F.Cu") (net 7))
 (segment (start 46.00 82.00) (end 46.00 80.00) (width 0.35) (layer "F.Cu") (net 7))
 (segment (start 46.00 82.00) (end 46.00 84.00) (width 0.35) (layer "F.Cu") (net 7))
 (segment (start 54.50 22.00) (end 53.00 22.00) (width 0.45) (layer "F.Cu") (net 8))
 (segment (start 53.00 22.00) (end 53.00 14.00) (width 0.45) (layer "F.Cu") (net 8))
 (segment (start 53.00 14.00) (end 60.00 14.00) (width 0.45) (layer "F.Cu") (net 8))
 (segment (start 60.00 14.00) (end 60.00 18.00) (width 0.45) (layer "F.Cu") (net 8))
 (segment (start 32.40 82.00) (end 32.40 84.00) (width 0.45) (layer "F.Cu") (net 8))
 (segment (start 32.40 84.00) (end 22.30 84.00) (width 0.45) (layer "F.Cu") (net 8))
 (segment (start 22.30 84.00) (end 22.30 78.00) (width 0.45) (layer "F.Cu") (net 8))
 (segment (start 18.00 43.40) (end 39.00 43.40) (width 0.20) (layer "F.Cu") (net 18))
 (segment (start 39.00 43.40) (end 39.00 24.00) (width 0.20) (layer "F.Cu") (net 18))
 (segment (start 39.00 24.00) (end 41.00 24.00) (width 0.20) (layer "F.Cu") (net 18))
 (segment (start 18.00 45.80) (end 41.00 45.80) (width 0.20) (layer "F.Cu") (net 19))
 (segment (start 41.00 45.80) (end 41.00 39.00) (width 0.20) (layer "F.Cu") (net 19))
 (segment (start 18.00 48.20) (end 30.00 48.20) (width 0.20) (layer "F.Cu") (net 20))
 (segment (start 30.00 48.20) (end 30.00 54.00) (width 0.20) (layer "F.Cu") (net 20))
 (segment (start 30.00 54.00) (end 41.00 54.00) (width 0.20) (layer "F.Cu") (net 20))
 (segment (start 34.80 82.00) (end 34.80 63.00) (width 0.20) (layer "F.Cu") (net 9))
 (segment (start 34.80 63.00) (end 38.00 61.00) (width 0.20) (layer "F.Cu") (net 9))
 (segment (start 37.20 82.00) (end 37.20 65.00) (width 0.20) (layer "F.Cu") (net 10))
 (segment (start 37.20 65.00) (end 38.00 63.40) (width 0.20) (layer "F.Cu") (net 10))
 (segment (start 39.60 82.00) (end 39.60 80.00) (width 0.20) (layer "F.Cu") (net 11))
 (segment (start 39.60 80.00) (end 44.00 80.00) (width 0.20) (layer "F.Cu") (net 11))
 (segment (start 40.80 82.00) (end 40.80 84.00) (width 0.20) (layer "F.Cu") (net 12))
 (segment (start 40.80 84.00) (end 44.00 84.00) (width 0.20) (layer "F.Cu") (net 12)))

